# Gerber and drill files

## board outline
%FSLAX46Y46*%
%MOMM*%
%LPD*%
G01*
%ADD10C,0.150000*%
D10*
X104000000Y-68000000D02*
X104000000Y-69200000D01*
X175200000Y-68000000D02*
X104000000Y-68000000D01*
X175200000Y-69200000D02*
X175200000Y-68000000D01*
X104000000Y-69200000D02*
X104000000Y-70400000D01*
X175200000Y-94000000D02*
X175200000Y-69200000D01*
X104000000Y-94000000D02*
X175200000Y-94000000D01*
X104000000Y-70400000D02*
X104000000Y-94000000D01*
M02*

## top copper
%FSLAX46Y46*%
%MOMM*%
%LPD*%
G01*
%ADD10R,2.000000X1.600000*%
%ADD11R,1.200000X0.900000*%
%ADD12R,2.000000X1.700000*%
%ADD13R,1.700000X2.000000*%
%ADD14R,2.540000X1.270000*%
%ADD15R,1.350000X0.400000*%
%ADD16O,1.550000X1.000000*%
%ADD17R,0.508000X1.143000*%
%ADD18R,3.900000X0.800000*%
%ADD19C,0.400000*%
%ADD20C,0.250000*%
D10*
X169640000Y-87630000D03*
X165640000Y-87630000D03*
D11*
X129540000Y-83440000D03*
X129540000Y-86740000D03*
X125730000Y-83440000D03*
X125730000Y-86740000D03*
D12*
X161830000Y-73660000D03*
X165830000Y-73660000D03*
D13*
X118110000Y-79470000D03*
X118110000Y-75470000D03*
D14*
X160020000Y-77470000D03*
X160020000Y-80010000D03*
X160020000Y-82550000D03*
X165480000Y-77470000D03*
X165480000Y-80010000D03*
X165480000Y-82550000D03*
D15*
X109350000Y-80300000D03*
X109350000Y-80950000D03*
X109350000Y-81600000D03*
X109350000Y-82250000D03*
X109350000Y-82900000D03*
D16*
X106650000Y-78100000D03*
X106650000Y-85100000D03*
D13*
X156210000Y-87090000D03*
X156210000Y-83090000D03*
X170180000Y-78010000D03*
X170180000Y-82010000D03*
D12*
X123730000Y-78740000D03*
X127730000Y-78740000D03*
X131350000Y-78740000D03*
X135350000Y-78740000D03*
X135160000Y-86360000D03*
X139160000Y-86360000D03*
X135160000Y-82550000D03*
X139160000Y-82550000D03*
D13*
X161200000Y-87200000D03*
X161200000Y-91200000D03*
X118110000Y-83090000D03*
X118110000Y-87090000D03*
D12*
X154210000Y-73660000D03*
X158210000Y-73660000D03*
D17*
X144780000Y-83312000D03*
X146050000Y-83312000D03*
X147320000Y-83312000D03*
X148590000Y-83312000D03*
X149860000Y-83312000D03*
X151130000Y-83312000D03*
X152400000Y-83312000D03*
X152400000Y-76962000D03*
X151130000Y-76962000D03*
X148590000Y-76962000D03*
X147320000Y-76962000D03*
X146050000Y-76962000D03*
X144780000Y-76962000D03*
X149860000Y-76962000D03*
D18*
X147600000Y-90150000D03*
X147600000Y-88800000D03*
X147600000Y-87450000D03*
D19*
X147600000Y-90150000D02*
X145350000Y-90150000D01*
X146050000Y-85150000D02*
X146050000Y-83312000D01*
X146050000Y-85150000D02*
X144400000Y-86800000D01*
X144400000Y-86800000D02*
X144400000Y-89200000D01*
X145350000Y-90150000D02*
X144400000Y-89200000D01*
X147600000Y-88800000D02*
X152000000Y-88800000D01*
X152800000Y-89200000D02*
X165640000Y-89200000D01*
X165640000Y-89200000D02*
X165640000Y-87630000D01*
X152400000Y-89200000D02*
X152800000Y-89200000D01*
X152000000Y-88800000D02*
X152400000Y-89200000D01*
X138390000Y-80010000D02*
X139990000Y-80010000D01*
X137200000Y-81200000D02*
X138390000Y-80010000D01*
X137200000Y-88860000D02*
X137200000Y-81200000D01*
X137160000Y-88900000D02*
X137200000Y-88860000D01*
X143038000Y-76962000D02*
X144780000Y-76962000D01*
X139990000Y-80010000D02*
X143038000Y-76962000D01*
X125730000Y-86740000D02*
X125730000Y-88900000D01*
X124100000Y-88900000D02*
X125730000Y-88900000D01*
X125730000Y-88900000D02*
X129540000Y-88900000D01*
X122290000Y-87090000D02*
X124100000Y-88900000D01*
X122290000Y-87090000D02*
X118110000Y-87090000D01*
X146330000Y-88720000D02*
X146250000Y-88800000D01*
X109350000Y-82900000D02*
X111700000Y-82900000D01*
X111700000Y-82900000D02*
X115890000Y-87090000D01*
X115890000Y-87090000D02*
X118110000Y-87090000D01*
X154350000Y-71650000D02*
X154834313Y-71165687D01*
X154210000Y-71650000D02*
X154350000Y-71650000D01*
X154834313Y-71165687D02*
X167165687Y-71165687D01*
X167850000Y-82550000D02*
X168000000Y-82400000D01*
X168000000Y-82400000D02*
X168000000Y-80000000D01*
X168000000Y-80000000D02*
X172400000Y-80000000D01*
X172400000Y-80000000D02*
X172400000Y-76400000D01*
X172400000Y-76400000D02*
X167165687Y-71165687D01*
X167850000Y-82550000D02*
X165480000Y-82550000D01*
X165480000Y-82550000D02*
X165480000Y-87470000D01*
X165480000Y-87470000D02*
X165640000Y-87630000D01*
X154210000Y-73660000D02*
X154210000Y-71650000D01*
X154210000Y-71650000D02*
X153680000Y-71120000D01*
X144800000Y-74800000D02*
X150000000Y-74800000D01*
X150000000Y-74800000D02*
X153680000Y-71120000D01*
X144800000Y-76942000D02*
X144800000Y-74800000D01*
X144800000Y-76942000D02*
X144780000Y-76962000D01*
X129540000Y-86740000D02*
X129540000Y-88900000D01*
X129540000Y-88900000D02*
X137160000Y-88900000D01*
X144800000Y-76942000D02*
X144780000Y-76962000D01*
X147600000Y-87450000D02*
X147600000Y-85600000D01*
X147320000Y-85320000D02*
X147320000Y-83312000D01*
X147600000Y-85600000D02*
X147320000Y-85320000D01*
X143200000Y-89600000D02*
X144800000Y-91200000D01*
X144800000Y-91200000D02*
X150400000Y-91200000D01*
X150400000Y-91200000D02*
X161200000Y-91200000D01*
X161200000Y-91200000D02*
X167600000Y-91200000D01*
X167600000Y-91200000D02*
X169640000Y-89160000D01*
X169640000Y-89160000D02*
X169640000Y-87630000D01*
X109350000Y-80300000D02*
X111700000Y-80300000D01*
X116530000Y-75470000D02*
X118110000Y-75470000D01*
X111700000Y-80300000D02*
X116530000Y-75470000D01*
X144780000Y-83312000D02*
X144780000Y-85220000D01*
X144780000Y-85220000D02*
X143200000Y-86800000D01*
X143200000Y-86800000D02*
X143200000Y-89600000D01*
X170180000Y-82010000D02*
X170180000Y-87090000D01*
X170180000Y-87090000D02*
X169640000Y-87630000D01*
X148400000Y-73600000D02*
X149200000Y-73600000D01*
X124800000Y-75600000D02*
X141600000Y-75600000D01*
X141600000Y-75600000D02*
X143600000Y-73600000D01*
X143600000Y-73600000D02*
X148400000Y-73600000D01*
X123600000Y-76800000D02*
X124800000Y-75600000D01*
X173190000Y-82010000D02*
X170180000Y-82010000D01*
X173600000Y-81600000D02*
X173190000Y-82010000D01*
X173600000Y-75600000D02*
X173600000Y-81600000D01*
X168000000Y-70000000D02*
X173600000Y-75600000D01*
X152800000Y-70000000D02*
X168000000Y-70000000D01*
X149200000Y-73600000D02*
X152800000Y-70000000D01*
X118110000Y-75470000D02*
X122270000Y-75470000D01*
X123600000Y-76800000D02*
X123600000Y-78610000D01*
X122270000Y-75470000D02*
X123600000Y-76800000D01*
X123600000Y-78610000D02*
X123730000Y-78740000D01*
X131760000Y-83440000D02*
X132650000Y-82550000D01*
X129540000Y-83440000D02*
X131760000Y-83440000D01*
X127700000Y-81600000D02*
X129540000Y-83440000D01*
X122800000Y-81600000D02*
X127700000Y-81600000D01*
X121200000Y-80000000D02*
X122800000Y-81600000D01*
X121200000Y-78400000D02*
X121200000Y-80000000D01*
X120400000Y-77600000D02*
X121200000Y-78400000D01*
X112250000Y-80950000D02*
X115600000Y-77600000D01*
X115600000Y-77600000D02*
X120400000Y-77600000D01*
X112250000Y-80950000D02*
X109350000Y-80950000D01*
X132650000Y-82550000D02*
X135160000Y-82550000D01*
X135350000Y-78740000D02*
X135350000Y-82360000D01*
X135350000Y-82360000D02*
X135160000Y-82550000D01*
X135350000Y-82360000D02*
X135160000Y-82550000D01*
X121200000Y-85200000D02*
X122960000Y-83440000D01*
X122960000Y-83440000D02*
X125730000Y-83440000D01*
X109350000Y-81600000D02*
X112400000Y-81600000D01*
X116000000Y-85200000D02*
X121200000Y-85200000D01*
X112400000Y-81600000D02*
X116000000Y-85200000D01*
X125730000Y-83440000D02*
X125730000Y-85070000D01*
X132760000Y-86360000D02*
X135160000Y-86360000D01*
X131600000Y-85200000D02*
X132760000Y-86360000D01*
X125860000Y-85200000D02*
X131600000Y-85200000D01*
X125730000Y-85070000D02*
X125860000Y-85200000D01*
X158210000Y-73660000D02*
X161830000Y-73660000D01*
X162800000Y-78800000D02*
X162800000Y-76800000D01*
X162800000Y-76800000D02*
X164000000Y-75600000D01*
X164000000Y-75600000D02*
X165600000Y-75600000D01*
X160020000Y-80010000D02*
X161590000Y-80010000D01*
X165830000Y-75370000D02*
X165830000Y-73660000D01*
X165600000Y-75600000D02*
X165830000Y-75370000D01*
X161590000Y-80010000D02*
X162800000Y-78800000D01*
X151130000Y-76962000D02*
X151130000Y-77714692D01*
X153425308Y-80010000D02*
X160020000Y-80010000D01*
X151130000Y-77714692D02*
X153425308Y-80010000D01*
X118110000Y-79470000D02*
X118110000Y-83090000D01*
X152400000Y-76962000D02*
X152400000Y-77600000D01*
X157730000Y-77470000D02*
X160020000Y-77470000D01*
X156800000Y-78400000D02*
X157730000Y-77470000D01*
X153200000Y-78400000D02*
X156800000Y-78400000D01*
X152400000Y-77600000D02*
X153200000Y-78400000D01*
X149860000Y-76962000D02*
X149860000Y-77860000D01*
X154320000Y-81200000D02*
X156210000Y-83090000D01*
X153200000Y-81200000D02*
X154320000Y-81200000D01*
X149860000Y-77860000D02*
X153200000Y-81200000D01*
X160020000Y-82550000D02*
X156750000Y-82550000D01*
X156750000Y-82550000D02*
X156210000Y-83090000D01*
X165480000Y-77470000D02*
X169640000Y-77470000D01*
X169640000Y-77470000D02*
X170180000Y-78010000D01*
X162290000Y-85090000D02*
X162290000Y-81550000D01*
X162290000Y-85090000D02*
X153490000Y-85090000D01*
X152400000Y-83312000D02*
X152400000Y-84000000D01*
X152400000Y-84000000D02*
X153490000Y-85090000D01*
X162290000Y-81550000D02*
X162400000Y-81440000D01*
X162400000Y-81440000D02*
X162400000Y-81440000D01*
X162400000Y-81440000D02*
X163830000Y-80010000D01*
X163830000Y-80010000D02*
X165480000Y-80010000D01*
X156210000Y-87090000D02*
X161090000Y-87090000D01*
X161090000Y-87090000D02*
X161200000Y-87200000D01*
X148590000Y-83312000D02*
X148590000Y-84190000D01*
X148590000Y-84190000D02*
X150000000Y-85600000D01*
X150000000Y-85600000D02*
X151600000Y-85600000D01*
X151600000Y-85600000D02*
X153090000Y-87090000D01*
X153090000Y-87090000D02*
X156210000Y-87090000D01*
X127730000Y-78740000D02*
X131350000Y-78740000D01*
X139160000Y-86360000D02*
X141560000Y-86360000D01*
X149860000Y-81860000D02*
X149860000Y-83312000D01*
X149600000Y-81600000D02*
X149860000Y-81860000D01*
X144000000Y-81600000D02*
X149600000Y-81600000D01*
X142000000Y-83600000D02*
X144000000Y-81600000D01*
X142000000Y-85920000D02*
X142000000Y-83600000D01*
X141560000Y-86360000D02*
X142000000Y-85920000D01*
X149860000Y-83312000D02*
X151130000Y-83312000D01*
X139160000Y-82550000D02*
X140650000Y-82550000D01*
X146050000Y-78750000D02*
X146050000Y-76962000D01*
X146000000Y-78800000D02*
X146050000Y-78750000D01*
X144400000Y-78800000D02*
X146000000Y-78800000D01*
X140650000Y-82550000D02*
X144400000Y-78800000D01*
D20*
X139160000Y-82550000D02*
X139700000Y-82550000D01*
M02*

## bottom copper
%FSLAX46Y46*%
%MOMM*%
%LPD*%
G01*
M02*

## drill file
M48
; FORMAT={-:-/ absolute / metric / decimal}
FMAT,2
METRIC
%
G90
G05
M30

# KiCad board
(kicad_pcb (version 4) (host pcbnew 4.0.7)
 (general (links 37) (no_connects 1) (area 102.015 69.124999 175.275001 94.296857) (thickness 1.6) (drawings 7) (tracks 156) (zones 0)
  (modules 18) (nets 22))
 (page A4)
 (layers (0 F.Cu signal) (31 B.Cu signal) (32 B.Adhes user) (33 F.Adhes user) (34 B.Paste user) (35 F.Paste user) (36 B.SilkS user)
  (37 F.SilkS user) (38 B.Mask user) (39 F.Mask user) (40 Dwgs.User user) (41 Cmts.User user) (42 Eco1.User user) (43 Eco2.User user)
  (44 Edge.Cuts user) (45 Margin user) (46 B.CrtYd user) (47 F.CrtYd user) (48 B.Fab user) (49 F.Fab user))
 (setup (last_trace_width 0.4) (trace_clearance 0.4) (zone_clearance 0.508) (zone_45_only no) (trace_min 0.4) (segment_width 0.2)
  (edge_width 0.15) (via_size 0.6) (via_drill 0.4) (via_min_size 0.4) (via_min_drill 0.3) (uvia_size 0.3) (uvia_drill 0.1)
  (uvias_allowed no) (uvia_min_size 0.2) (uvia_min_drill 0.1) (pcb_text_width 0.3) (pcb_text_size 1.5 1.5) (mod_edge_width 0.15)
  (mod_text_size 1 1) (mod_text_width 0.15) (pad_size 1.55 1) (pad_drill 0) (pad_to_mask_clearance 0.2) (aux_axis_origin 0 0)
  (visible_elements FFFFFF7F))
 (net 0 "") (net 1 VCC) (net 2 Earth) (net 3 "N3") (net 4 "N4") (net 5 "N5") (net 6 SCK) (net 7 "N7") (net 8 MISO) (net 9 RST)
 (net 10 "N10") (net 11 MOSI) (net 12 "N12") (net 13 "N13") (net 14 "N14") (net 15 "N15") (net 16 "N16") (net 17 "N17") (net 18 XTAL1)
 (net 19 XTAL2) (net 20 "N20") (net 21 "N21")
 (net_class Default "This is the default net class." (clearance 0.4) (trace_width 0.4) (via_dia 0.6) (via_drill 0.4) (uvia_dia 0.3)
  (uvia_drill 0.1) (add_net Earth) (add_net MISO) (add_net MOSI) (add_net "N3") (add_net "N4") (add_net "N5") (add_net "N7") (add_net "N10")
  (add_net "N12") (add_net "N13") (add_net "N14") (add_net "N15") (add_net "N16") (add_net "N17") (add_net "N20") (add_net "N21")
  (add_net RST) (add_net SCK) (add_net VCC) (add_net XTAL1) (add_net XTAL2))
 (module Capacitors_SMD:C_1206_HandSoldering (layer F.Cu) (at 167.64 87.63 180)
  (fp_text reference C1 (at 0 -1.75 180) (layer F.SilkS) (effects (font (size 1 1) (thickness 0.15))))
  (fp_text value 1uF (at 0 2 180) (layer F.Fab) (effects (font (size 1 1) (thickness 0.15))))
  (pad 1 smd rect (at -2 0 180) (size 2 1.6) (layers F.Cu F.Paste F.Mask) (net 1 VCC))
  (pad 2 smd rect (at 2 0 180) (size 2 1.6) (layers F.Cu F.Paste F.Mask) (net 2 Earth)))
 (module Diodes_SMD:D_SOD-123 (layer F.Cu) (at 129.54 85.09 270)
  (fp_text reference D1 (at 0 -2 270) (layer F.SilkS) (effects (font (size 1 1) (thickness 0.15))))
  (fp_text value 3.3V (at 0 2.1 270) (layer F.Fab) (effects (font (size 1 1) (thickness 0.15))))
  (pad 1 smd rect (at -1.65 0 270) (size 0.9 1.2) (layers F.Cu F.Paste F.Mask) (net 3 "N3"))
  (pad 2 smd rect (at 1.65 0 270) (size 0.9 1.2) (layers F.Cu F.Paste F.Mask) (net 2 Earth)))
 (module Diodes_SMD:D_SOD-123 (layer F.Cu) (at 125.73 85.09 270)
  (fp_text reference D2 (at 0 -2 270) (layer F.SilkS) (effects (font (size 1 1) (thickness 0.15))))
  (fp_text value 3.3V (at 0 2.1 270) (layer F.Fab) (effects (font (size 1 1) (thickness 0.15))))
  (pad 1 smd rect (at -1.65 0 270) (size 0.9 1.2) (layers F.Cu F.Paste F.Mask) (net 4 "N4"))
  (pad 2 smd rect (at 1.65 0 270) (size 0.9 1.2) (layers F.Cu F.Paste F.Mask) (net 2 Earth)))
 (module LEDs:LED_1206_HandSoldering (layer F.Cu) (at 163.83 73.66)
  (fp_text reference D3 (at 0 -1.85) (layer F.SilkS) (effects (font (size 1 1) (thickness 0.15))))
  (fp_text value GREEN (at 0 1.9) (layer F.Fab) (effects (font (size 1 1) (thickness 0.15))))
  (pad 1 smd rect (at -2 0) (size 2 1.7) (layers F.Cu F.Paste F.Mask) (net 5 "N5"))
  (pad 2 smd rect (at 2 0) (size 2 1.7) (layers F.Cu F.Paste F.Mask) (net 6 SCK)))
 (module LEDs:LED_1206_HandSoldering (layer F.Cu) (at 118.11 77.47 90)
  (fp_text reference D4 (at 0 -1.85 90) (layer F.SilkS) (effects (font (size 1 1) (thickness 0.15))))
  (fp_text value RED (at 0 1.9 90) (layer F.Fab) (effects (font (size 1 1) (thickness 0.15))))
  (pad 1 smd rect (at -2 0 90) (size 2 1.7) (layers F.Cu F.Paste F.Mask) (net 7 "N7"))
  (pad 2 smd rect (at 2 0 90) (size 2 1.7) (layers F.Cu F.Paste F.Mask) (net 1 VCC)))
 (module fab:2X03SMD (layer F.Cu) (at 162.56 80.01)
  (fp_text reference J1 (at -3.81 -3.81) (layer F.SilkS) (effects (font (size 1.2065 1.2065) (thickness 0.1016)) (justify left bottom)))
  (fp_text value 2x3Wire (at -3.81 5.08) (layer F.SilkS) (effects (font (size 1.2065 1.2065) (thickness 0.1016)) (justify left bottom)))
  (pad 1 smd rect (at -2.54 -2.54) (size 2.54 1.27) (layers F.Cu F.Paste F.Mask) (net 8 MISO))
  (pad 3 smd rect (at -2.54 0) (size 2.54 1.27) (layers F.Cu F.Paste F.Mask) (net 6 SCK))
  (pad 5 smd rect (at -2.54 2.54) (size 2.54 1.27) (layers F.Cu F.Paste F.Mask) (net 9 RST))
  (pad 2 smd rect (at 2.92 -2.54) (size 2.54 1.27) (layers F.Cu F.Paste F.Mask) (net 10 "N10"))
  (pad 4 smd rect (at 2.92 0) (size 2.54 1.27) (layers F.Cu F.Paste F.Mask) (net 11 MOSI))
  (pad 6 smd rect (at 2.92 2.54) (size 2.54 1.27) (layers F.Cu F.Paste F.Mask) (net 2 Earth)))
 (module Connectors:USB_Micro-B (layer F.Cu) (at 108 81.6 270)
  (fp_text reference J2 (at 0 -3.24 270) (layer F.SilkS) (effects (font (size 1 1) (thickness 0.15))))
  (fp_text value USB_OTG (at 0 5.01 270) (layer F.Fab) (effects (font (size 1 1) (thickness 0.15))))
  (pad 1 smd rect (at -1.3 -1.35) (size 1.35 0.4) (layers F.Cu F.Paste F.Mask) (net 1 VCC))
  (pad 2 smd rect (at -0.65 -1.35) (size 1.35 0.4) (layers F.Cu F.Paste F.Mask) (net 3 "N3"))
  (pad 3 smd rect (at 0 -1.35) (size 1.35 0.4) (layers F.Cu F.Paste F.Mask) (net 4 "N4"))
  (pad 4 smd rect (at 0.65 -1.35) (size 1.35 0.4) (layers F.Cu F.Paste F.Mask) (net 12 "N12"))
  (pad 5 smd rect (at 1.3 -1.35) (size 1.35 0.4) (layers F.Cu F.Paste F.Mask) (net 2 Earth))
  (pad 6 smd oval (at -3.5 1.35) (size 1.55 1) (layers F.Cu F.Paste F.Mask) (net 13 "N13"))
  (pad 6 smd oval (at 3.5 1.35) (size 1.55 1) (layers F.Cu F.Paste F.Mask) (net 13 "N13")))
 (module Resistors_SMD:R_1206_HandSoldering (layer F.Cu) (at 156.21 85.09 90)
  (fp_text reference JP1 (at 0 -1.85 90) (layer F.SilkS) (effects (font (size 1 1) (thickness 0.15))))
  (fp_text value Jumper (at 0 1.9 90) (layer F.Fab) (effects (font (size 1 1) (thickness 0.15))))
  (pad 1 smd rect (at -2 0 90) (size 2 1.7) (layers F.Cu F.Paste F.Mask) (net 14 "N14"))
  (pad 2 smd rect (at 2 0 90) (size 2 1.7) (layers F.Cu F.Paste F.Mask) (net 9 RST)))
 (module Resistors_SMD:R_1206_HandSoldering (layer F.Cu) (at 170.18 80.01 270)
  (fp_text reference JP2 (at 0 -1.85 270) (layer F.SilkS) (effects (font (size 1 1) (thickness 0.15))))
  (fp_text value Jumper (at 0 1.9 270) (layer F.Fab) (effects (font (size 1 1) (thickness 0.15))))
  (pad 1 smd rect (at -2 0 270) (size 2 1.7) (layers F.Cu F.Paste F.Mask) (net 10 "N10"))
  (pad 2 smd rect (at 2 0 270) (size 2 1.7) (layers F.Cu F.Paste F.Mask) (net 1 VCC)))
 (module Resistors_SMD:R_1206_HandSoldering (layer F.Cu) (at 125.73 78.74)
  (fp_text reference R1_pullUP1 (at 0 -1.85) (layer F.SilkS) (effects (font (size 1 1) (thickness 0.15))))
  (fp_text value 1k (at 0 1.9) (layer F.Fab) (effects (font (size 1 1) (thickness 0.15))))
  (pad 1 smd rect (at -2 0) (size 2 1.7) (layers F.Cu F.Paste F.Mask) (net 1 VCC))
  (pad 2 smd rect (at 2 0) (size 2 1.7) (layers F.Cu F.Paste F.Mask) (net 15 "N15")))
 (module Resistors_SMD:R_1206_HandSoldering (layer F.Cu) (at 133.35 78.74)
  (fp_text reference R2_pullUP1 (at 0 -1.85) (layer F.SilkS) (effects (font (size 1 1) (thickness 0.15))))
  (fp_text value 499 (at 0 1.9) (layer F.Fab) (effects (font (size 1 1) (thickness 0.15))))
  (pad 1 smd rect (at -2 0) (size 2 1.7) (layers F.Cu F.Paste F.Mask) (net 15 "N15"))
  (pad 2 smd rect (at 2 0) (size 2 1.7) (layers F.Cu F.Paste F.Mask) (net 3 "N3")))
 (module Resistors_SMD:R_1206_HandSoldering (layer F.Cu) (at 137.16 86.36)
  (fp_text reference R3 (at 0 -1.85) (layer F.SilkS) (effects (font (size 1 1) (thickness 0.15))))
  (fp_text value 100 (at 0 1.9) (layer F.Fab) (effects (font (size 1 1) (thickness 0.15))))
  (pad 1 smd rect (at -2 0) (size 2 1.7) (layers F.Cu F.Paste F.Mask) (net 4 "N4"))
  (pad 2 smd rect (at 2 0) (size 2 1.7) (layers F.Cu F.Paste F.Mask) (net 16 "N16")))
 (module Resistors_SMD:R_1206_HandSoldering (layer F.Cu) (at 137.16 82.55)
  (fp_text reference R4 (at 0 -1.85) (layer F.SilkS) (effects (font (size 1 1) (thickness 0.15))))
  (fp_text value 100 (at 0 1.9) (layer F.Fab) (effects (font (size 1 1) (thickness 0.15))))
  (pad 1 smd rect (at -2 0) (size 2 1.7) (layers F.Cu F.Paste F.Mask) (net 3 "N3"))
  (pad 2 smd rect (at 2 0) (size 2 1.7) (layers F.Cu F.Paste F.Mask) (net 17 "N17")))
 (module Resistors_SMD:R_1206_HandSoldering (layer F.Cu) (at 161.2 89.2 270)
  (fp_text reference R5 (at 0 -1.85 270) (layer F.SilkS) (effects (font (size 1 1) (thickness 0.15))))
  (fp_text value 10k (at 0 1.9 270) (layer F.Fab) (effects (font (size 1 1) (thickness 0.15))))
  (pad 1 smd rect (at -2 0 270) (size 2 1.7) (layers F.Cu F.Paste F.Mask) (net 14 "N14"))
  (pad 2 smd rect (at 2 0 270) (size 2 1.7) (layers F.Cu F.Paste F.Mask) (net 1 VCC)))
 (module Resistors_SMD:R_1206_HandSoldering (layer F.Cu) (at 118.11 85.09 270)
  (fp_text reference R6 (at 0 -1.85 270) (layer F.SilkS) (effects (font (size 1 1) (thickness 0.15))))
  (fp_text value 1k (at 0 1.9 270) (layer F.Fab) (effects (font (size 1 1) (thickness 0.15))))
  (pad 1 smd rect (at -2 0 270) (size 2 1.7) (layers F.Cu F.Paste F.Mask) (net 7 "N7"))
  (pad 2 smd rect (at 2 0 270) (size 2 1.7) (layers F.Cu F.Paste F.Mask) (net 2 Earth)))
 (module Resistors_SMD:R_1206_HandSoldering (layer F.Cu) (at 156.21 73.66)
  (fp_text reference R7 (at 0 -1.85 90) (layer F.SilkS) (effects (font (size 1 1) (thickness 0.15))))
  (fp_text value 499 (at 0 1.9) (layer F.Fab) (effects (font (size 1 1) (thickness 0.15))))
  (pad 1 smd rect (at -2 0) (size 2 1.7) (layers F.Cu F.Paste F.Mask) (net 2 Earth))
  (pad 2 smd rect (at 2 0) (size 2 1.7) (layers F.Cu F.Paste F.Mask) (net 5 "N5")))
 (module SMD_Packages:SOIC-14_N (layer F.Cu) (at 148.59 80.01)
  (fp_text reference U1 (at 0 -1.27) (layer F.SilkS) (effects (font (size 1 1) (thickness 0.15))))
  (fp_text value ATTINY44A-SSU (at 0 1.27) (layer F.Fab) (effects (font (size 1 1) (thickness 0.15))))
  (pad 1 smd rect (at -3.81 3.302) (size 0.508 1.143) (layers F.Cu F.Paste F.Mask) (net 1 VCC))
  (pad 2 smd rect (at -2.54 3.302) (size 0.508 1.143) (layers F.Cu F.Paste F.Mask) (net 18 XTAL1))
  (pad 3 smd rect (at -1.27 3.302) (size 0.508 1.143) (layers F.Cu F.Paste F.Mask) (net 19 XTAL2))
  (pad 4 smd rect (at 0 3.302) (size 0.508 1.143) (layers F.Cu F.Paste F.Mask) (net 14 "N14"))
  (pad 5 smd rect (at 1.27 3.302) (size 0.508 1.143) (layers F.Cu F.Paste F.Mask) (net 16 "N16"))
  (pad 6 smd rect (at 2.54 3.302) (size 0.508 1.143) (layers F.Cu F.Paste F.Mask) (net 16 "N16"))
  (pad 7 smd rect (at 3.81 3.302) (size 0.508 1.143) (layers F.Cu F.Paste F.Mask) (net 11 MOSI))
  (pad 8 smd rect (at 3.81 -3.048) (size 0.508 1.143) (layers F.Cu F.Paste F.Mask) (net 8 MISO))
  (pad 9 smd rect (at 2.54 -3.048) (size 0.508 1.143) (layers F.Cu F.Paste F.Mask) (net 6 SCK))
  (pad 11 smd rect (at 0 -3.048) (size 0.508 1.143) (layers F.Cu F.Paste F.Mask) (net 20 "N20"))
  (pad 12 smd rect (at -1.27 -3.048) (size 0.508 1.143) (layers F.Cu F.Paste F.Mask) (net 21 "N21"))
  (pad 13 smd rect (at -2.54 -3.048) (size 0.508 1.143) (layers F.Cu F.Paste F.Mask) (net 17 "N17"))
  (pad 14 smd rect (at -3.81 -3.048) (size 0.508 1.143) (layers F.Cu F.Paste F.Mask) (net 2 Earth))
  (pad 10 smd rect (at 1.27 -3.048) (size 0.508 1.143) (layers F.Cu F.Paste F.Mask) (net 9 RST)))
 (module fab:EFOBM (layer F.Cu) (at 147.6 88.8 90)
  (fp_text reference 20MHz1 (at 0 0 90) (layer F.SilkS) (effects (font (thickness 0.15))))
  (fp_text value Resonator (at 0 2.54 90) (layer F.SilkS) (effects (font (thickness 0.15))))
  (pad 1 smd rect (at -1.35 0 180) (size 3.9 0.8) (layers F.Cu F.Paste F.Mask) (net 18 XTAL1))
  (pad 2 smd rect (at 0 0) (size 3.9 0.8) (layers F.Cu F.Paste F.Mask) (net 2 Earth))
  (pad 3 smd rect (at 1.35 0) (size 3.9 0.8) (layers F.Cu F.Paste F.Mask) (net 19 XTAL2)))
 (gr_line (start 104 68) (end 104 69.2) (angle 90) (layer Edge.Cuts) (width 0.15))
 (gr_line (start 175.2 68) (end 104 68) (angle 90) (layer Edge.Cuts) (width 0.15))
 (gr_line (start 175.2 69.2) (end 175.2 68) (angle 90) (layer Edge.Cuts) (width 0.15))
 (gr_line (start 104 69.2) (end 104 70.4) (angle 90) (layer Edge.Cuts) (width 0.15))
 (gr_line (start 175.2 94) (end 175.2 69.2) (angle 90) (layer Edge.Cuts) (width 0.15))
 (gr_line (start 104 94) (end 175.2 94) (angle 90) (layer Edge.Cuts) (width 0.15))
 (gr_line (start 104 70.4) (end 104 94) (angle 90) (layer Edge.Cuts) (width 0.15))
 (segment (start 147.6 90.15) (end 145.35 90.15) (width 0.4) (layer F.Cu) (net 18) (status 400000))
 (segment (start 146.05 85.15) (end 146.05 83.312) (width 0.4) (layer F.Cu) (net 18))
 (segment (start 146.05 85.15) (end 144.4 86.8) (width 0.4) (layer F.Cu) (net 18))
 (segment (start 144.4 86.8) (end 144.4 89.2) (width 0.4) (layer F.Cu) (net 18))
 (segment (start 145.35 90.15) (end 144.4 89.2) (width 0.4) (layer F.Cu) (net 18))
 (segment (start 147.6 88.8) (end 152 88.8) (width 0.4) (layer F.Cu) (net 2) (status 400000))
 (segment (start 152.8 89.2) (end 165.64 89.2) (width 0.4) (layer F.Cu) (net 2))
 (segment (start 165.64 89.2) (end 165.64 87.63) (width 0.4) (layer F.Cu) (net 2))
 (segment (start 152.4 89.2) (end 152.8 89.2) (width 0.4) (layer F.Cu) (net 2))
 (segment (start 152 88.8) (end 152.4 89.2) (width 0.4) (layer F.Cu) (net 2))
 (segment (start 138.39 80.01) (end 139.99 80.01) (width 0.4) (layer F.Cu) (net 2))
 (segment (start 137.2 81.2) (end 138.39 80.01) (width 0.4) (layer F.Cu) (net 2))
 (segment (start 137.2 88.86) (end 137.2 81.2) (width 0.4) (layer F.Cu) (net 2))
 (segment (start 137.16 88.9) (end 137.2 88.86) (width 0.4) (layer F.Cu) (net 2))
 (segment (start 143.038 76.962) (end 144.78 76.962) (width 0.4) (layer F.Cu) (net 2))
 (segment (start 139.99 80.01) (end 143.038 76.962) (width 0.4) (layer F.Cu) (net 2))
 (segment (start 125.73 86.74) (end 125.73 88.9) (width 0.4) (layer F.Cu) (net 2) (status 10))
 (segment (start 124.1 88.9) (end 125.73 88.9) (width 0.4) (layer F.Cu) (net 2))
 (segment (start 125.73 88.9) (end 129.54 88.9) (width 0.4) (layer F.Cu) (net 2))
 (segment (start 122.29 87.09) (end 124.1 88.9) (width 0.4) (layer F.Cu) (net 2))
 (segment (start 122.29 87.09) (end 118.11 87.09) (width 0.4) (layer F.Cu) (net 2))
 (segment (start 146.33 88.72) (end 146.25 88.8) (width 0.4) (layer F.Cu) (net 2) (status 30))
 (segment (start 109.35 82.9) (end 111.7 82.9) (width 0.4) (layer F.Cu) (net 2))
 (segment (start 111.7 82.9) (end 115.89 87.09) (width 0.4) (layer F.Cu) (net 2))
 (segment (start 115.89 87.09) (end 118.11 87.09) (width 0.4) (layer F.Cu) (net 2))
 (segment (start 154.35 71.65) (end 154.834313 71.165687) (width 0.4) (layer F.Cu) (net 2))
 (segment (start 154.21 71.65) (end 154.35 71.65) (width 0.4) (layer F.Cu) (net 2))
 (segment (start 154.834313 71.165687) (end 167.165687 71.165687) (width 0.4) (layer F.Cu) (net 2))
 (segment (start 167.85 82.55) (end 168 82.4) (width 0.4) (layer F.Cu) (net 2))
 (segment (start 168 82.4) (end 168 80) (width 0.4) (layer F.Cu) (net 2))
 (segment (start 168 80) (end 172.4 80) (width 0.4) (layer F.Cu) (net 2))
 (segment (start 172.4 80) (end 172.4 76.4) (width 0.4) (layer F.Cu) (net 2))
 (segment (start 172.4 76.4) (end 167.165687 71.165687) (width 0.4) (layer F.Cu) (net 2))
 (segment (start 167.85 82.55) (end 165.48 82.55) (width 0.4) (layer F.Cu) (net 2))
 (segment (start 165.48 82.55) (end 165.48 87.47) (width 0.4) (layer F.Cu) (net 2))
 (segment (start 165.48 87.47) (end 165.64 87.63) (width 0.4) (layer F.Cu) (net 2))
 (segment (start 154.21 73.66) (end 154.21 71.65) (width 0.4) (layer F.Cu) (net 2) (status 10))
 (segment (start 154.21 71.65) (end 153.68 71.12) (width 0.4) (layer F.Cu) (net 2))
 (segment (start 144.8 74.8) (end 150 74.8) (width 0.4) (layer F.Cu) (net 2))
 (segment (start 150 74.8) (end 153.68 71.12) (width 0.4) (layer F.Cu) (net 2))
 (segment (start 144.8 76.942) (end 144.8 74.8) (width 0.4) (layer F.Cu) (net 2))
 (segment (start 144.8 76.942) (end 144.78 76.962) (width 0.4) (layer F.Cu) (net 2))
 (segment (start 129.54 86.74) (end 129.54 88.9) (width 0.4) (layer F.Cu) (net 2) (status 10))
 (segment (start 129.54 88.9) (end 137.16 88.9) (width 0.4) (layer F.Cu) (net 2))
 (segment (start 144.8 76.942) (end 144.78 76.962) (width 0.4) (layer F.Cu) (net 2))
 (segment (start 147.6 87.45) (end 147.6 85.6) (width 0.4) (layer F.Cu) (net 19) (status 400000))
 (segment (start 147.32 85.32) (end 147.32 83.312) (width 0.4) (layer F.Cu) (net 19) (status 800000))
 (segment (start 147.6 85.6) (end 147.32 85.32) (width 0.4) (layer F.Cu) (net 19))
 (segment (start 143.2 89.6) (end 144.8 91.2) (width 0.4) (layer F.Cu) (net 1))
 (segment (start 144.8 91.2) (end 150.4 91.2) (width 0.4) (layer F.Cu) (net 1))
 (segment (start 150.4 91.2) (end 161.2 91.2) (width 0.4) (layer F.Cu) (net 1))
 (segment (start 161.2 91.2) (end 167.6 91.2) (width 0.4) (layer F.Cu) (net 1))
 (segment (start 167.6 91.2) (end 169.64 89.16) (width 0.4) (layer F.Cu) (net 1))
 (segment (start 169.64 89.16) (end 169.64 87.63) (width 0.4) (layer F.Cu) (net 1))
 (segment (start 109.35 80.3) (end 111.7 80.3) (width 0.4) (layer F.Cu) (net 1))
 (segment (start 116.53 75.47) (end 118.11 75.47) (width 0.4) (layer F.Cu) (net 1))
 (segment (start 111.7 80.3) (end 116.53 75.47) (width 0.4) (layer F.Cu) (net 1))
 (segment (start 144.78 83.312) (end 144.78 85.22) (width 0.4) (layer F.Cu) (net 1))
 (segment (start 144.78 85.22) (end 143.2 86.8) (width 0.4) (layer F.Cu) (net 1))
 (segment (start 143.2 86.8) (end 143.2 89.6) (width 0.4) (layer F.Cu) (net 1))
 (segment (start 170.18 82.01) (end 170.18 87.09) (width 0.4) (layer F.Cu) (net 1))
 (segment (start 170.18 87.09) (end 169.64 87.63) (width 0.4) (layer F.Cu) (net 1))
 (segment (start 148.4 73.6) (end 149.2 73.6) (width 0.4) (layer F.Cu) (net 1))
 (segment (start 124.8 75.6) (end 141.6 75.6) (width 0.4) (layer F.Cu) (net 1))
 (segment (start 141.6 75.6) (end 143.6 73.6) (width 0.4) (layer F.Cu) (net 1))
 (segment (start 143.6 73.6) (end 148.4 73.6) (width 0.4) (layer F.Cu) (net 1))
 (segment (start 123.6 76.8) (end 124.8 75.6) (width 0.4) (layer F.Cu) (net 1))
 (segment (start 173.19 82.01) (end 170.18 82.01) (width 0.4) (layer F.Cu) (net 1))
 (segment (start 173.6 81.6) (end 173.19 82.01) (width 0.4) (layer F.Cu) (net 1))
 (segment (start 173.6 75.6) (end 173.6 81.6) (width 0.4) (layer F.Cu) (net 1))
 (segment (start 168 70) (end 173.6 75.6) (width 0.4) (layer F.Cu) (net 1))
 (segment (start 152.8 70) (end 168 70) (width 0.4) (layer F.Cu) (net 1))
 (segment (start 149.2 73.6) (end 152.8 70) (width 0.4) (layer F.Cu) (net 1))
 (segment (start 118.11 75.47) (end 122.27 75.47) (width 0.4) (layer F.Cu) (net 1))
 (segment (start 123.6 76.8) (end 123.6 78.61) (width 0.4) (layer F.Cu) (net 1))
 (segment (start 122.27 75.47) (end 123.6 76.8) (width 0.4) (layer F.Cu) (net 1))
 (segment (start 123.6 78.61) (end 123.73 78.74) (width 0.4) (layer F.Cu) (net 1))
 (segment (start 131.76 83.44) (end 132.65 82.55) (width 0.4) (layer F.Cu) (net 3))
 (segment (start 129.54 83.44) (end 131.76 83.44) (width 0.4) (layer F.Cu) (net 3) (status 10))
 (segment (start 127.7 81.6) (end 129.54 83.44) (width 0.4) (layer F.Cu) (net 3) (status 20))
 (segment (start 122.8 81.6) (end 127.7 81.6) (width 0.4) (layer F.Cu) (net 3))
 (segment (start 121.2 80) (end 122.8 81.6) (width 0.4) (layer F.Cu) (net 3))
 (segment (start 121.2 78.4) (end 121.2 80) (width 0.4) (layer F.Cu) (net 3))
 (segment (start 120.4 77.6) (end 121.2 78.4) (width 0.4) (layer F.Cu) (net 3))
 (segment (start 112.25 80.95) (end 115.6 77.6) (width 0.4) (layer F.Cu) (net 3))
 (segment (start 115.6 77.6) (end 120.4 77.6) (width 0.4) (layer F.Cu) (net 3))
 (segment (start 112.25 80.95) (end 109.35 80.95) (width 0.4) (layer F.Cu) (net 3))
 (segment (start 132.65 82.55) (end 135.16 82.55) (width 0.4) (layer F.Cu) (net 3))
 (segment (start 135.35 78.74) (end 135.35 82.36) (width 0.4) (layer F.Cu) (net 3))
 (segment (start 135.35 82.36) (end 135.16 82.55) (width 0.4) (layer F.Cu) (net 3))
 (segment (start 135.35 82.36) (end 135.16 82.55) (width 0.4) (layer F.Cu) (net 3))
 (segment (start 121.2 85.2) (end 122.96 83.44) (width 0.4) (layer F.Cu) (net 4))
 (segment (start 122.96 83.44) (end 125.73 83.44) (width 0.4) (layer F.Cu) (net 4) (status 20))
 (segment (start 109.35 81.6) (end 112.4 81.6) (width 0.4) (layer F.Cu) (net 4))
 (segment (start 116 85.2) (end 121.2 85.2) (width 0.4) (layer F.Cu) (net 4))
 (segment (start 112.4 81.6) (end 116 85.2) (width 0.4) (layer F.Cu) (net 4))
 (segment (start 125.73 83.44) (end 125.73 85.07) (width 0.4) (layer F.Cu) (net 4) (status 10))
 (segment (start 132.76 86.36) (end 135.16 86.36) (width 0.4) (layer F.Cu) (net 4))
 (segment (start 131.6 85.2) (end 132.76 86.36) (width 0.4) (layer F.Cu) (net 4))
 (segment (start 125.86 85.2) (end 131.6 85.2) (width 0.4) (layer F.Cu) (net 4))
 (segment (start 125.73 85.07) (end 125.86 85.2) (width 0.4) (layer F.Cu) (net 4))
 (segment (start 158.21 73.66) (end 161.83 73.66) (width 0.4) (layer F.Cu) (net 5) (status 20))
 (segment (start 162.8 78.8) (end 162.8 76.8) (width 0.4) (layer F.Cu) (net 6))
 (segment (start 162.8 76.8) (end 164 75.6) (width 0.4) (layer F.Cu) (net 6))
 (segment (start 164 75.6) (end 165.6 75.6) (width 0.4) (layer F.Cu) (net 6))
 (segment (start 160.02 80.01) (end 161.59 80.01) (width 0.4) (layer F.Cu) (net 6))
 (segment (start 165.83 75.37) (end 165.83 73.66) (width 0.4) (layer F.Cu) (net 6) (status 20))
 (segment (start 165.6 75.6) (end 165.83 75.37) (width 0.4) (layer F.Cu) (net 6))
 (segment (start 161.59 80.01) (end 162.8 78.8) (width 0.4) (layer F.Cu) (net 6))
 (segment (start 151.13 76.962) (end 151.13 77.714692) (width 0.4) (layer F.Cu) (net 6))
 (segment (start 153.425308 80.01) (end 160.02 80.01) (width 0.4) (layer F.Cu) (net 6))
 (segment (start 151.13 77.714692) (end 153.425308 80.01) (width 0.4) (layer F.Cu) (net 6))
 (segment (start 118.11 79.47) (end 118.11 83.09) (width 0.4) (layer F.Cu) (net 7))
 (segment (start 152.4 76.962) (end 152.4 77.6) (width 0.4) (layer F.Cu) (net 8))
 (segment (start 157.73 77.47) (end 160.02 77.47) (width 0.4) (layer F.Cu) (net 8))
 (segment (start 156.8 78.4) (end 157.73 77.47) (width 0.4) (layer F.Cu) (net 8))
 (segment (start 153.2 78.4) (end 156.8 78.4) (width 0.4) (layer F.Cu) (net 8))
 (segment (start 152.4 77.6) (end 153.2 78.4) (width 0.4) (layer F.Cu) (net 8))
 (segment (start 149.86 76.962) (end 149.86 77.86) (width 0.4) (layer F.Cu) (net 9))
 (segment (start 154.32 81.2) (end 156.21 83.09) (width 0.4) (layer F.Cu) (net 9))
 (segment (start 153.2 81.2) (end 154.32 81.2) (width 0.4) (layer F.Cu) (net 9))
 (segment (start 149.86 77.86) (end 153.2 81.2) (width 0.4) (layer F.Cu) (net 9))
 (segment (start 160.02 82.55) (end 156.75 82.55) (width 0.4) (layer F.Cu) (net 9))
 (segment (start 156.75 82.55) (end 156.21 83.09) (width 0.4) (layer F.Cu) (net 9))
 (segment (start 165.48 77.47) (end 169.64 77.47) (width 0.4) (layer F.Cu) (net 10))
 (segment (start 169.64 77.47) (end 170.18 78.01) (width 0.4) (layer F.Cu) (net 10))
 (segment (start 162.29 85.09) (end 162.29 81.55) (width 0.4) (layer F.Cu) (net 11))
 (segment (start 162.29 85.09) (end 153.49 85.09) (width 0.4) (layer F.Cu) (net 11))
 (segment (start 152.4 83.312) (end 152.4 84) (width 0.4) (layer F.Cu) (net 11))
 (segment (start 152.4 84) (end 153.49 85.09) (width 0.4) (layer F.Cu) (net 11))
 (segment (start 162.29 81.55) (end 162.4 81.44) (width 0.4) (layer F.Cu) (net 11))
 (segment (start 162.4 81.44) (end 162.4 81.44) (width 0.4) (layer F.Cu) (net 11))
 (segment (start 162.4 81.44) (end 163.83 80.01) (width 0.4) (layer F.Cu) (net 11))
 (segment (start 163.83 80.01) (end 165.48 80.01) (width 0.4) (layer F.Cu) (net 11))
 (segment (start 156.21 87.09) (end 161.09 87.09) (width 0.4) (layer F.Cu) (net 14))
 (segment (start 161.09 87.09) (end 161.2 87.2) (width 0.4) (layer F.Cu) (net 14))
 (segment (start 148.59 83.312) (end 148.59 84.19) (width 0.4) (layer F.Cu) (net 14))
 (segment (start 148.59 84.19) (end 150 85.6) (width 0.4) (layer F.Cu) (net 14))
 (segment (start 150 85.6) (end 151.6 85.6) (width 0.4) (layer F.Cu) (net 14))
 (segment (start 151.6 85.6) (end 153.09 87.09) (width 0.4) (layer F.Cu) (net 14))
 (segment (start 153.09 87.09) (end 156.21 87.09) (width 0.4) (layer F.Cu) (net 14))
 (segment (start 127.73 78.74) (end 131.35 78.74) (width 0.4) (layer F.Cu) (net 15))
 (segment (start 139.16 86.36) (end 141.56 86.36) (width 0.4) (layer F.Cu) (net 16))
 (segment (start 149.86 81.86) (end 149.86 83.312) (width 0.4) (layer F.Cu) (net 16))
 (segment (start 149.6 81.6) (end 149.86 81.86) (width 0.4) (layer F.Cu) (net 16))
 (segment (start 144 81.6) (end 149.6 81.6) (width 0.4) (layer F.Cu) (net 16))
 (segment (start 142 83.6) (end 144 81.6) (width 0.4) (layer F.Cu) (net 16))
 (segment (start 142 85.92) (end 142 83.6) (width 0.4) (layer F.Cu) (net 16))
 (segment (start 141.56 86.36) (end 142 85.92) (width 0.4) (layer F.Cu) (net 16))
 (segment (start 149.86 83.312) (end 151.13 83.312) (width 0.4) (layer F.Cu) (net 16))
 (segment (start 139.16 82.55) (end 140.65 82.55) (width 0.4) (layer F.Cu) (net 17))
 (segment (start 146.05 78.75) (end 146.05 76.962) (width 0.4) (layer F.Cu) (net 17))
 (segment (start 146 78.8) (end 146.05 78.75) (width 0.4) (layer F.Cu) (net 17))
 (segment (start 144.4 78.8) (end 146 78.8) (width 0.4) (layer F.Cu) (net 17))
 (segment (start 140.65 82.55) (end 144.4 78.8) (width 0.4) (layer F.Cu) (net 17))
 (segment (start 139.16 82.55) (end 139.7 82.55) (width 0.25) (layer F.Cu) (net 17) (status 30)))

